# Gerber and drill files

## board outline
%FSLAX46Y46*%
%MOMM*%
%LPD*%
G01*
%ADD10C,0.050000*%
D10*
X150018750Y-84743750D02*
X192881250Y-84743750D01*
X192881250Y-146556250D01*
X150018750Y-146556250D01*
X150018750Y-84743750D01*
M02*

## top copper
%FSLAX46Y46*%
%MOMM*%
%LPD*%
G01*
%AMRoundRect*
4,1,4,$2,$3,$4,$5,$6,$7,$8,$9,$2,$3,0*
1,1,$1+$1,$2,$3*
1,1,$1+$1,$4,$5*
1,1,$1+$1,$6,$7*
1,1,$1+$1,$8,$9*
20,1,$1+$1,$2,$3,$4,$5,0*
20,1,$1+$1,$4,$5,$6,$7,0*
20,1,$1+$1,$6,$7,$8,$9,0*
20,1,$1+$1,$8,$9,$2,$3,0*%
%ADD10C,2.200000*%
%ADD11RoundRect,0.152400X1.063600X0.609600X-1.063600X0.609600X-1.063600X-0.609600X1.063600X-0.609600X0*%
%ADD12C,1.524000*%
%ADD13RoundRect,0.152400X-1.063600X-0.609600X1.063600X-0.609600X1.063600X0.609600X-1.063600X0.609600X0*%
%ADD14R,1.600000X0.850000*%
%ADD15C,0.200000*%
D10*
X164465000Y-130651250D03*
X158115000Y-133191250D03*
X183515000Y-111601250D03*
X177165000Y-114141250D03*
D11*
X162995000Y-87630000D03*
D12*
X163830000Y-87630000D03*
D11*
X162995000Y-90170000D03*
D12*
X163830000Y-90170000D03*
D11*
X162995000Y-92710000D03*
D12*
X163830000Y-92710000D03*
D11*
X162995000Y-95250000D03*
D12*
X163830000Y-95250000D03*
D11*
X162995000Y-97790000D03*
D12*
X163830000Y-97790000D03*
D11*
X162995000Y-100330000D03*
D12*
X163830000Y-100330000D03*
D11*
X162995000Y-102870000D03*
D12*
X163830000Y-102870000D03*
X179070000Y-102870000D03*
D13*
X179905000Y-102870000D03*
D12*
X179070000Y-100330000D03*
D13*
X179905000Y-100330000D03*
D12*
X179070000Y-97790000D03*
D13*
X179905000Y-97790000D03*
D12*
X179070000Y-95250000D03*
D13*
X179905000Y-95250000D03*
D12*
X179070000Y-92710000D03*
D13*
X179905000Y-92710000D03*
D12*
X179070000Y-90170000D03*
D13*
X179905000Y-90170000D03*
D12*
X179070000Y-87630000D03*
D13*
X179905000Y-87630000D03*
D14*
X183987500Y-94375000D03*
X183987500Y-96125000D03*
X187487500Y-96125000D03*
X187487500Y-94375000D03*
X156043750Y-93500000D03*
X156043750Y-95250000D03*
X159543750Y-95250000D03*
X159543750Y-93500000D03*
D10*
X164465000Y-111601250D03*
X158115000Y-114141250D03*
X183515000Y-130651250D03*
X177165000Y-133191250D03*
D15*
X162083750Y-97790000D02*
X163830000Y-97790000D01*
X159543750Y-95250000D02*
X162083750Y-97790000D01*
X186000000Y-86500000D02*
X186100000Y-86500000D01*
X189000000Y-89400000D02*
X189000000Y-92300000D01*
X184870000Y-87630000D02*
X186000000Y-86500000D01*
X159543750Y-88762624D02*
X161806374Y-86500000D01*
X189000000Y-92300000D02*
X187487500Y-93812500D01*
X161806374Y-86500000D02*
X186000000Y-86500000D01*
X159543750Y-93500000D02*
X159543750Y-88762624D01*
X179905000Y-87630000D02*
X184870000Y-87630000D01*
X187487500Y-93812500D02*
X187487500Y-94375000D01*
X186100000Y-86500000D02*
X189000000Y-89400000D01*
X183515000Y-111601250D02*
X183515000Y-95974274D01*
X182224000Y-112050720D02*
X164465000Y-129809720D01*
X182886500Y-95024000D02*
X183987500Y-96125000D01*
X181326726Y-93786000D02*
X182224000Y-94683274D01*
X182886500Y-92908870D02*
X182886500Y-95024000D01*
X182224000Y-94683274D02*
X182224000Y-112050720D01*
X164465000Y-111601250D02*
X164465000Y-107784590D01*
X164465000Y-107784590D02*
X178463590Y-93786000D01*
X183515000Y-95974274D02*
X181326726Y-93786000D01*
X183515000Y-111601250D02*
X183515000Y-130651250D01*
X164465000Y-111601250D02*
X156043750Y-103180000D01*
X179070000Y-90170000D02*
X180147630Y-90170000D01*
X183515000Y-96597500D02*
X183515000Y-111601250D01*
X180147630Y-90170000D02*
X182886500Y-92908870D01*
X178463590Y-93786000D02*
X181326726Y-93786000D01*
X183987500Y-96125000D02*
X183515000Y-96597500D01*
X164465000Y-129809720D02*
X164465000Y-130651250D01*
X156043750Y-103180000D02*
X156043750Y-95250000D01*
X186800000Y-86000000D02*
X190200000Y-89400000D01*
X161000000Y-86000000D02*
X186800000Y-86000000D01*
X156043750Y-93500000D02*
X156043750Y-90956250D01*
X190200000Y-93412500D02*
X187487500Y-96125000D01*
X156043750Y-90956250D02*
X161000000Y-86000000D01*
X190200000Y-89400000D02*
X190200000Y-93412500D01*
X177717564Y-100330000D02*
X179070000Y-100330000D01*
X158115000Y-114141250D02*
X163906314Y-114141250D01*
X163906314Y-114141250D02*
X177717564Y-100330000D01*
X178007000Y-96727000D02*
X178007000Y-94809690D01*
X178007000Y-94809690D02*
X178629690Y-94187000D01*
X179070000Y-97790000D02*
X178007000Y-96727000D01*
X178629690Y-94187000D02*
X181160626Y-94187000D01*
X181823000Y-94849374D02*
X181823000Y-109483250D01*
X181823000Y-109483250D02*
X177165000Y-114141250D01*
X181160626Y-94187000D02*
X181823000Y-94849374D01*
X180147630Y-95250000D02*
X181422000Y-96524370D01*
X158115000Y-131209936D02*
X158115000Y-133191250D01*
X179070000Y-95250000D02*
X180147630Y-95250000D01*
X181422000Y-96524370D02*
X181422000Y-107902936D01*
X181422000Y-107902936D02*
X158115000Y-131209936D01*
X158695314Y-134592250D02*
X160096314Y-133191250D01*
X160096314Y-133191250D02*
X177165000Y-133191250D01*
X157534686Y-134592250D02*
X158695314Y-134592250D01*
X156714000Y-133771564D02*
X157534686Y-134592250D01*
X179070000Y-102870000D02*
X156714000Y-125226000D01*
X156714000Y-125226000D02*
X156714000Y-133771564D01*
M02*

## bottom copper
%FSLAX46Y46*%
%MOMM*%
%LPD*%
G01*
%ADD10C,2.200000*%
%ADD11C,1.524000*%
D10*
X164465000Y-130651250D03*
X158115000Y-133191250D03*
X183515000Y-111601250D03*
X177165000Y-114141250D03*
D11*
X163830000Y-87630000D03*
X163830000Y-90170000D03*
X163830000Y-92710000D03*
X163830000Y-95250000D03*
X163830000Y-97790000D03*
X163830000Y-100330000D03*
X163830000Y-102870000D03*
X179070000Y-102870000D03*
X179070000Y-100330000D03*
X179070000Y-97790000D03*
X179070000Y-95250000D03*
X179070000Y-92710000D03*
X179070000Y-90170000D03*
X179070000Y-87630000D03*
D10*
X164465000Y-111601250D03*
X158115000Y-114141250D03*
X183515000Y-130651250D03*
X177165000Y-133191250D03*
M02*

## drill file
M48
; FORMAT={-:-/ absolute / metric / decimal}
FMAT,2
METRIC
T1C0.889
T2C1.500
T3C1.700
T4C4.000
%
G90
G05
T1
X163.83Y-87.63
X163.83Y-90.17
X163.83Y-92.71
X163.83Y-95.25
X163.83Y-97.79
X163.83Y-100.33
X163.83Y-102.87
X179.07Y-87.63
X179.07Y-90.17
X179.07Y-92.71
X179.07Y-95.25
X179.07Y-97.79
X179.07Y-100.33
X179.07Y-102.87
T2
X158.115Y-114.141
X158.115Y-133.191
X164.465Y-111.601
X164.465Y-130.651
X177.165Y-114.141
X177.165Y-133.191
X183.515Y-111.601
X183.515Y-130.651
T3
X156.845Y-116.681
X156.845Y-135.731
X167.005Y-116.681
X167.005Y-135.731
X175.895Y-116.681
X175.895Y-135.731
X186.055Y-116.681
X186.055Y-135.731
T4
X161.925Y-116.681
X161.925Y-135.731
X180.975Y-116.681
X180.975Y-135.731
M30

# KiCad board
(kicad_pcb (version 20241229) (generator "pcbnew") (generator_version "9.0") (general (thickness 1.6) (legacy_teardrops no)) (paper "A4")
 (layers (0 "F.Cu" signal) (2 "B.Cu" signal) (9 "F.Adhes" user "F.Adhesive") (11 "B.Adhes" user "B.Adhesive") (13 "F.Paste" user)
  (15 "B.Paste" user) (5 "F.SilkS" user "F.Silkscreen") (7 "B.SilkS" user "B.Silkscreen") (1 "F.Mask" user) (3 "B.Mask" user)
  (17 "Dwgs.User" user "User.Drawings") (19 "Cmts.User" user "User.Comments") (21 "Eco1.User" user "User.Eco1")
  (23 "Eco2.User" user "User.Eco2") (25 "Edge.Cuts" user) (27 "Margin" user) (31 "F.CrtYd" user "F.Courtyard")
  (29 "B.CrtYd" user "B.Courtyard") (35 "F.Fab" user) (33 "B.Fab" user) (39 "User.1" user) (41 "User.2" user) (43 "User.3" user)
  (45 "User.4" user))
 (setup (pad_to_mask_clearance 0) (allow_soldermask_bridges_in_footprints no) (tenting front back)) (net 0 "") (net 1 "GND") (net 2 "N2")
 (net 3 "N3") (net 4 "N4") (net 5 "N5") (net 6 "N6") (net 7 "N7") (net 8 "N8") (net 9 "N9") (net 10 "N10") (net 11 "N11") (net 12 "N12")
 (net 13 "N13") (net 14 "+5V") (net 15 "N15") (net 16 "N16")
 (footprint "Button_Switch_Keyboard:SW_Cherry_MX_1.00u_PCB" (layer "F.Cu") (at 164.465 130.65125)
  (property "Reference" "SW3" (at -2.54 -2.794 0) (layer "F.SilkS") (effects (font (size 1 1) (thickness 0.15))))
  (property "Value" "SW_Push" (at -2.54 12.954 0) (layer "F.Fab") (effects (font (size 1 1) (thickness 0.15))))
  (pad "" np_thru_hole circle (at -7.62 5.08) (size 1.7 1.7) (drill 1.7) (layers "*.Cu" "*.Mask"))
  (pad "" np_thru_hole circle (at -2.54 5.08) (size 4 4) (drill 4) (layers "*.Cu" "*.Mask"))
  (pad "" np_thru_hole circle (at 2.54 5.08) (size 1.7 1.7) (drill 1.7) (layers "*.Cu" "*.Mask"))
  (pad "1" thru_hole circle (at 0 0) (size 2.2 2.2) (drill 1.5) (layers "*.Cu" "*.Mask") (remove_unused_layers no) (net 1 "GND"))
  (pad "2" thru_hole circle (at -6.35 2.54) (size 2.2 2.2) (drill 1.5) (layers "*.Cu" "*.Mask") (remove_unused_layers no) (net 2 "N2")))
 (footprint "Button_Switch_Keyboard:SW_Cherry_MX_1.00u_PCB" (layer "F.Cu") (at 183.515 111.60125)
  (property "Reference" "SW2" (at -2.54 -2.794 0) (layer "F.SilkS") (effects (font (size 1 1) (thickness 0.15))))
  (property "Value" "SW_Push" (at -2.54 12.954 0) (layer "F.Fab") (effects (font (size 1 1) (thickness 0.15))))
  (pad "" np_thru_hole circle (at -7.62 5.08) (size 1.7 1.7) (drill 1.7) (layers "*.Cu" "*.Mask"))
  (pad "" np_thru_hole circle (at -2.54 5.08) (size 4 4) (drill 4) (layers "*.Cu" "*.Mask"))
  (pad "" np_thru_hole circle (at 2.54 5.08) (size 1.7 1.7) (drill 1.7) (layers "*.Cu" "*.Mask"))
  (pad "1" thru_hole circle (at 0 0) (size 2.2 2.2) (drill 1.5) (layers "*.Cu" "*.Mask") (remove_unused_layers no) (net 1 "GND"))
  (pad "2" thru_hole circle (at -6.35 2.54) (size 2.2 2.2) (drill 1.5) (layers "*.Cu" "*.Mask") (remove_unused_layers no) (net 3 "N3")))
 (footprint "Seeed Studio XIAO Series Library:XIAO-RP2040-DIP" (layer "F.Cu") (at 171.45 95.25)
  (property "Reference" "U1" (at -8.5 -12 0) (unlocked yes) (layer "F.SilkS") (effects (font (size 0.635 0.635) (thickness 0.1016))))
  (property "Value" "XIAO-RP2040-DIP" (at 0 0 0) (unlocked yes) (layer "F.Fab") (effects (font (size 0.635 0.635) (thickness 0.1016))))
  (pad "1" smd roundrect (at -8.455 -7.62 180) (size 2.432 1.524) (layers "F.Cu" "F.Mask") (roundrect_rratio 0.1) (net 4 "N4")
   (thermal_bridge_angle 45))
  (pad "1" thru_hole circle (at -7.62 -7.62 180) (size 1.524 1.524) (drill 0.889) (layers "*.Cu" "*.Mask") (remove_unused_layers no)
   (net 4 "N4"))
  (pad "2" smd roundrect (at -8.455 -5.08 180) (size 2.432 1.524) (layers "F.Cu" "F.Mask") (roundrect_rratio 0.1) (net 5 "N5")
   (thermal_bridge_angle 45))
  (pad "2" thru_hole circle (at -7.62 -5.08 180) (size 1.524 1.524) (drill 0.889) (layers "*.Cu" "*.Mask") (remove_unused_layers no)
   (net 5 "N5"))
  (pad "3" smd roundrect (at -8.455 -2.54 180) (size 2.432 1.524) (layers "F.Cu" "F.Mask") (roundrect_rratio 0.1) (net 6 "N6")
   (thermal_bridge_angle 45))
  (pad "3" thru_hole circle (at -7.62 -2.54 180) (size 1.524 1.524) (drill 0.889) (layers "*.Cu" "*.Mask") (remove_unused_layers no)
   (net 6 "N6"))
  (pad "4" smd roundrect (at -8.455 0 180) (size 2.432 1.524) (layers "F.Cu" "F.Mask") (roundrect_rratio 0.1) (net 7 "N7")
   (thermal_bridge_angle 45))
  (pad "4" thru_hole circle (at -7.62 0 180) (size 1.524 1.524) (drill 0.889) (layers "*.Cu" "*.Mask") (remove_unused_layers no)
   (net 7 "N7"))
  (pad "5" smd roundrect (at -8.455 2.54 180) (size 2.432 1.524) (layers "F.Cu" "F.Mask") (roundrect_rratio 0.1) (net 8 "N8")
   (thermal_bridge_angle 45))
  (pad "5" thru_hole circle (at -7.62 2.54 180) (size 1.524 1.524) (drill 0.889) (layers "*.Cu" "*.Mask") (remove_unused_layers no)
   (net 8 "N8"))
  (pad "6" smd roundrect (at -8.455 5.08 180) (size 2.432 1.524) (layers "F.Cu" "F.Mask") (roundrect_rratio 0.1) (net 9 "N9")
   (thermal_bridge_angle 45))
  (pad "6" thru_hole circle (at -7.62 5.08 180) (size 1.524 1.524) (drill 0.889) (layers "*.Cu" "*.Mask") (remove_unused_layers no)
   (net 9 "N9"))
  (pad "7" smd roundrect (at -8.455 7.62 180) (size 2.432 1.524) (layers "F.Cu" "F.Mask") (roundrect_rratio 0.1) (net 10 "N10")
   (thermal_bridge_angle 45))
  (pad "7" thru_hole circle (at -7.62 7.62 180) (size 1.524 1.524) (drill 0.889) (layers "*.Cu" "*.Mask") (remove_unused_layers no)
   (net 10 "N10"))
  (pad "8" thru_hole circle (at 7.62 7.62) (size 1.524 1.524) (drill 0.889) (layers "*.Cu" "*.Mask") (remove_unused_layers no)
   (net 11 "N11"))
  (pad "8" smd roundrect (at 8.455 7.62) (size 2.432 1.524) (layers "F.Cu" "F.Mask") (roundrect_rratio 0.1) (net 11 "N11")
   (thermal_bridge_angle 45))
  (pad "9" thru_hole circle (at 7.62 5.08) (size 1.524 1.524) (drill 0.889) (layers "*.Cu" "*.Mask") (remove_unused_layers no)
   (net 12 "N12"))
  (pad "9" smd roundrect (at 8.455 5.08) (size 2.432 1.524) (layers "F.Cu" "F.Mask") (roundrect_rratio 0.1) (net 12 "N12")
   (thermal_bridge_angle 45))
  (pad "10" thru_hole circle (at 7.62 2.54) (size 1.524 1.524) (drill 0.889) (layers "*.Cu" "*.Mask") (remove_unused_layers no) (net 3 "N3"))
  (pad "10" smd roundrect (at 8.455 2.54) (size 2.432 1.524) (layers "F.Cu" "F.Mask") (roundrect_rratio 0.1) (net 3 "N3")
   (thermal_bridge_angle 45))
  (pad "11" thru_hole circle (at 7.62 0) (size 1.524 1.524) (drill 0.889) (layers "*.Cu" "*.Mask") (remove_unused_layers no) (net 2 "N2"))
  (pad "11" smd roundrect (at 8.455 0) (size 2.432 1.524) (layers "F.Cu" "F.Mask") (roundrect_rratio 0.1) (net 2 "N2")
   (thermal_bridge_angle 45))
  (pad "12" thru_hole circle (at 7.62 -2.54) (size 1.524 1.524) (drill 0.889) (layers "*.Cu" "*.Mask") (remove_unused_layers no)
   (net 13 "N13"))
  (pad "12" smd roundrect (at 8.455 -2.54) (size 2.432 1.524) (layers "F.Cu" "F.Mask") (roundrect_rratio 0.1) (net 13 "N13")
   (thermal_bridge_angle 45))
  (pad "13" thru_hole circle (at 7.62 -5.08) (size 1.524 1.524) (drill 0.889) (layers "*.Cu" "*.Mask") (remove_unused_layers no)
   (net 1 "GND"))
  (pad "13" smd roundrect (at 8.455 -5.08) (size 2.432 1.524) (layers "F.Cu" "F.Mask") (roundrect_rratio 0.1) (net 1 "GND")
   (thermal_bridge_angle 45))
  (pad "14" thru_hole circle (at 7.62 -7.62) (size 1.524 1.524) (drill 0.889) (layers "*.Cu" "*.Mask") (remove_unused_layers no)
   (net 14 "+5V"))
  (pad "14" smd roundrect (at 8.455 -7.62) (size 2.432 1.524) (layers "F.Cu" "F.Mask") (roundrect_rratio 0.1) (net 14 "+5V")
   (thermal_bridge_angle 45)))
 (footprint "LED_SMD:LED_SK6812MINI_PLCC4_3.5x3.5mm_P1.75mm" (layer "F.Cu") (at 185.7375 95.25)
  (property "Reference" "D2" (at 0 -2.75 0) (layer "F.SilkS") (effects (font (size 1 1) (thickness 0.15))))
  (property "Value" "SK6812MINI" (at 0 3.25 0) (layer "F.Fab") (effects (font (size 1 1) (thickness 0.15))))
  (pad "1" smd rect (at -1.75 -0.875) (size 1.6 0.85) (layers "F.Cu" "F.Mask" "F.Paste") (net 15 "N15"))
  (pad "2" smd rect (at -1.75 0.875) (size 1.6 0.85) (layers "F.Cu" "F.Mask" "F.Paste") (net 1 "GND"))
  (pad "3" smd rect (at 1.75 0.875) (size 1.6 0.85) (layers "F.Cu" "F.Mask" "F.Paste") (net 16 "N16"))
  (pad "4" smd rect (at 1.75 -0.875) (size 1.6 0.85) (layers "F.Cu" "F.Mask" "F.Paste") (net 14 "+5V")))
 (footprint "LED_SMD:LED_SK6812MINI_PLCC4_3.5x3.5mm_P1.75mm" (layer "F.Cu") (at 157.79375 94.375)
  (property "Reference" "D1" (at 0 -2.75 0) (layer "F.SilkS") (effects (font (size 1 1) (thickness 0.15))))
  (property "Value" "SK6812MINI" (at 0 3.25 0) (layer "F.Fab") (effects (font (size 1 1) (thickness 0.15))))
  (pad "1" smd rect (at -1.75 -0.875) (size 1.6 0.85) (layers "F.Cu" "F.Mask" "F.Paste") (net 16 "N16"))
  (pad "2" smd rect (at -1.75 0.875) (size 1.6 0.85) (layers "F.Cu" "F.Mask" "F.Paste") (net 1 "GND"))
  (pad "3" smd rect (at 1.75 0.875) (size 1.6 0.85) (layers "F.Cu" "F.Mask" "F.Paste") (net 8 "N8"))
  (pad "4" smd rect (at 1.75 -0.875) (size 1.6 0.85) (layers "F.Cu" "F.Mask" "F.Paste") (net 14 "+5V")))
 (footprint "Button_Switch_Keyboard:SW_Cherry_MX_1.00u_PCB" (layer "F.Cu") (at 164.465 111.60125)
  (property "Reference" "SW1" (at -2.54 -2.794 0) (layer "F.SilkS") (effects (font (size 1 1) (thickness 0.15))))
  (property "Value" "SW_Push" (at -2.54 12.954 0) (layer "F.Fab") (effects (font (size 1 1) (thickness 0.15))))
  (pad "" np_thru_hole circle (at -7.62 5.08) (size 1.7 1.7) (drill 1.7) (layers "*.Cu" "*.Mask"))
  (pad "" np_thru_hole circle (at -2.54 5.08) (size 4 4) (drill 4) (layers "*.Cu" "*.Mask"))
  (pad "" np_thru_hole circle (at 2.54 5.08) (size 1.7 1.7) (drill 1.7) (layers "*.Cu" "*.Mask"))
  (pad "1" thru_hole circle (at 0 0) (size 2.2 2.2) (drill 1.5) (layers "*.Cu" "*.Mask") (remove_unused_layers no) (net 1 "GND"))
  (pad "2" thru_hole circle (at -6.35 2.54) (size 2.2 2.2) (drill 1.5) (layers "*.Cu" "*.Mask") (remove_unused_layers no) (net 12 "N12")))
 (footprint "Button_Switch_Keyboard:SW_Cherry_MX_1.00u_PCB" (layer "F.Cu") (at 183.515 130.65125)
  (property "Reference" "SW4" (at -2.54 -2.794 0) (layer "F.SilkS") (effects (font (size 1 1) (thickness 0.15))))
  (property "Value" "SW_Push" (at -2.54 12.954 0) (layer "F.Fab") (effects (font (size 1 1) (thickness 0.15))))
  (pad "" np_thru_hole circle (at -7.62 5.08) (size 1.7 1.7) (drill 1.7) (layers "*.Cu" "*.Mask"))
  (pad "" np_thru_hole circle (at -2.54 5.08) (size 4 4) (drill 4) (layers "*.Cu" "*.Mask"))
  (pad "" np_thru_hole circle (at 2.54 5.08) (size 1.7 1.7) (drill 1.7) (layers "*.Cu" "*.Mask"))
  (pad "1" thru_hole circle (at 0 0) (size 2.2 2.2) (drill 1.5) (layers "*.Cu" "*.Mask") (remove_unused_layers no) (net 1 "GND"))
  (pad "2" thru_hole circle (at -6.35 2.54) (size 2.2 2.2) (drill 1.5) (layers "*.Cu" "*.Mask") (remove_unused_layers no) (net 11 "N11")))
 (gr_rect (start 150.01875 84.74375) (end 192.88125 146.55625) (stroke (width 0.05) (type default)) (fill no) (layer "Edge.Cuts"))
 (segment (start 162.08375 97.79) (end 163.83 97.79) (width 0.2) (layer "F.Cu") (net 8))
 (segment (start 159.54375 95.25) (end 162.08375 97.79) (width 0.2) (layer "F.Cu") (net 8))
 (segment (start 186 86.5) (end 186.1 86.5) (width 0.2) (layer "F.Cu") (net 14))
 (segment (start 189 89.4) (end 189 92.3) (width 0.2) (layer "F.Cu") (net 14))
 (segment (start 184.87 87.63) (end 186 86.5) (width 0.2) (layer "F.Cu") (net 14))
 (segment (start 159.54375 88.762624) (end 161.806374 86.5) (width 0.2) (layer "F.Cu") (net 14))
 (segment (start 189 92.3) (end 187.4875 93.8125) (width 0.2) (layer "F.Cu") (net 14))
 (segment (start 161.806374 86.5) (end 186 86.5) (width 0.2) (layer "F.Cu") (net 14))
 (segment (start 159.54375 93.5) (end 159.54375 88.762624) (width 0.2) (layer "F.Cu") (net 14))
 (segment (start 179.905 87.63) (end 184.87 87.63) (width 0.2) (layer "F.Cu") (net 14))
 (segment (start 187.4875 93.8125) (end 187.4875 94.375) (width 0.2) (layer "F.Cu") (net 14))
 (segment (start 186.1 86.5) (end 189 89.4) (width 0.2) (layer "F.Cu") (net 14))
 (segment (start 183.515 111.60125) (end 183.515 95.974274) (width 0.2) (layer "F.Cu") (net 1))
 (segment (start 182.224 112.05072) (end 164.465 129.80972) (width 0.2) (layer "F.Cu") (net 1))
 (segment (start 182.8865 95.024) (end 183.9875 96.125) (width 0.2) (layer "F.Cu") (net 1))
 (segment (start 181.326726 93.786) (end 182.224 94.683274) (width 0.2) (layer "F.Cu") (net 1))
 (segment (start 182.8865 92.90887) (end 182.8865 95.024) (width 0.2) (layer "F.Cu") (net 1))
 (segment (start 182.224 94.683274) (end 182.224 112.05072) (width 0.2) (layer "F.Cu") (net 1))
 (segment (start 164.465 111.60125) (end 164.465 107.78459) (width 0.2) (layer "F.Cu") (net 1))
 (segment (start 164.465 107.78459) (end 178.46359 93.786) (width 0.2) (layer "F.Cu") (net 1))
 (segment (start 183.515 95.974274) (end 181.326726 93.786) (width 0.2) (layer "F.Cu") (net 1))
 (segment (start 183.515 111.60125) (end 183.515 130.65125) (width 0.2) (layer "F.Cu") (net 1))
 (segment (start 164.465 111.60125) (end 156.04375 103.18) (width 0.2) (layer "F.Cu") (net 1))
 (segment (start 179.07 90.17) (end 180.14763 90.17) (width 0.2) (layer "F.Cu") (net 1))
 (segment (start 183.515 96.5975) (end 183.515 111.60125) (width 0.2) (layer "F.Cu") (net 1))
 (segment (start 180.14763 90.17) (end 182.8865 92.90887) (width 0.2) (layer "F.Cu") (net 1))
 (segment (start 178.46359 93.786) (end 181.326726 93.786) (width 0.2) (layer "F.Cu") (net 1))
 (segment (start 183.9875 96.125) (end 183.515 96.5975) (width 0.2) (layer "F.Cu") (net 1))
 (segment (start 164.465 129.80972) (end 164.465 130.65125) (width 0.2) (layer "F.Cu") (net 1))
 (segment (start 156.04375 103.18) (end 156.04375 95.25) (width 0.2) (layer "F.Cu") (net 1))
 (segment (start 186.8 86) (end 190.2 89.4) (width 0.2) (layer "F.Cu") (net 16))
 (segment (start 161 86) (end 186.8 86) (width 0.2) (layer "F.Cu") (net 16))
 (segment (start 156.04375 93.5) (end 156.04375 90.95625) (width 0.2) (layer "F.Cu") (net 16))
 (segment (start 190.2 93.4125) (end 187.4875 96.125) (width 0.2) (layer "F.Cu") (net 16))
 (segment (start 156.04375 90.95625) (end 161 86) (width 0.2) (layer "F.Cu") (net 16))
 (segment (start 190.2 89.4) (end 190.2 93.4125) (width 0.2) (layer "F.Cu") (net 16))
 (segment (start 177.717564 100.33) (end 179.07 100.33) (width 0.2) (layer "F.Cu") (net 12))
 (segment (start 158.115 114.14125) (end 163.906314 114.14125) (width 0.2) (layer "F.Cu") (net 12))
 (segment (start 163.906314 114.14125) (end 177.717564 100.33) (width 0.2) (layer "F.Cu") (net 12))
 (segment (start 178.007 96.727) (end 178.007 94.80969) (width 0.2) (layer "F.Cu") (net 3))
 (segment (start 178.007 94.80969) (end 178.62969 94.187) (width 0.2) (layer "F.Cu") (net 3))
 (segment (start 179.07 97.79) (end 178.007 96.727) (width 0.2) (layer "F.Cu") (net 3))
 (segment (start 178.62969 94.187) (end 181.160626 94.187) (width 0.2) (layer "F.Cu") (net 3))
 (segment (start 181.823 94.849374) (end 181.823 109.48325) (width 0.2) (layer "F.Cu") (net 3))
 (segment (start 181.823 109.48325) (end 177.165 114.14125) (width 0.2) (layer "F.Cu") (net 3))
 (segment (start 181.160626 94.187) (end 181.823 94.849374) (width 0.2) (layer "F.Cu") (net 3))
 (segment (start 180.14763 95.25) (end 181.422 96.52437) (width 0.2) (layer "F.Cu") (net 2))
 (segment (start 158.115 131.209936) (end 158.115 133.19125) (width 0.2) (layer "F.Cu") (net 2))
 (segment (start 179.07 95.25) (end 180.14763 95.25) (width 0.2) (layer "F.Cu") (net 2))
 (segment (start 181.422 96.52437) (end 181.422 107.902936) (width 0.2) (layer "F.Cu") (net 2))
 (segment (start 181.422 107.902936) (end 158.115 131.209936) (width 0.2) (layer "F.Cu") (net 2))
 (segment (start 158.695314 134.59225) (end 160.096314 133.19125) (width 0.2) (layer "F.Cu") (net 11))
 (segment (start 160.096314 133.19125) (end 177.165 133.19125) (width 0.2) (layer "F.Cu") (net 11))
 (segment (start 157.534686 134.59225) (end 158.695314 134.59225) (width 0.2) (layer "F.Cu") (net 11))
 (segment (start 156.714 133.771564) (end 157.534686 134.59225) (width 0.2) (layer "F.Cu") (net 11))
 (segment (start 179.07 102.87) (end 156.714 125.226) (width 0.2) (layer "F.Cu") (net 11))
 (segment (start 156.714 125.226) (end 156.714 133.771564) (width 0.2) (layer "F.Cu") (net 11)))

